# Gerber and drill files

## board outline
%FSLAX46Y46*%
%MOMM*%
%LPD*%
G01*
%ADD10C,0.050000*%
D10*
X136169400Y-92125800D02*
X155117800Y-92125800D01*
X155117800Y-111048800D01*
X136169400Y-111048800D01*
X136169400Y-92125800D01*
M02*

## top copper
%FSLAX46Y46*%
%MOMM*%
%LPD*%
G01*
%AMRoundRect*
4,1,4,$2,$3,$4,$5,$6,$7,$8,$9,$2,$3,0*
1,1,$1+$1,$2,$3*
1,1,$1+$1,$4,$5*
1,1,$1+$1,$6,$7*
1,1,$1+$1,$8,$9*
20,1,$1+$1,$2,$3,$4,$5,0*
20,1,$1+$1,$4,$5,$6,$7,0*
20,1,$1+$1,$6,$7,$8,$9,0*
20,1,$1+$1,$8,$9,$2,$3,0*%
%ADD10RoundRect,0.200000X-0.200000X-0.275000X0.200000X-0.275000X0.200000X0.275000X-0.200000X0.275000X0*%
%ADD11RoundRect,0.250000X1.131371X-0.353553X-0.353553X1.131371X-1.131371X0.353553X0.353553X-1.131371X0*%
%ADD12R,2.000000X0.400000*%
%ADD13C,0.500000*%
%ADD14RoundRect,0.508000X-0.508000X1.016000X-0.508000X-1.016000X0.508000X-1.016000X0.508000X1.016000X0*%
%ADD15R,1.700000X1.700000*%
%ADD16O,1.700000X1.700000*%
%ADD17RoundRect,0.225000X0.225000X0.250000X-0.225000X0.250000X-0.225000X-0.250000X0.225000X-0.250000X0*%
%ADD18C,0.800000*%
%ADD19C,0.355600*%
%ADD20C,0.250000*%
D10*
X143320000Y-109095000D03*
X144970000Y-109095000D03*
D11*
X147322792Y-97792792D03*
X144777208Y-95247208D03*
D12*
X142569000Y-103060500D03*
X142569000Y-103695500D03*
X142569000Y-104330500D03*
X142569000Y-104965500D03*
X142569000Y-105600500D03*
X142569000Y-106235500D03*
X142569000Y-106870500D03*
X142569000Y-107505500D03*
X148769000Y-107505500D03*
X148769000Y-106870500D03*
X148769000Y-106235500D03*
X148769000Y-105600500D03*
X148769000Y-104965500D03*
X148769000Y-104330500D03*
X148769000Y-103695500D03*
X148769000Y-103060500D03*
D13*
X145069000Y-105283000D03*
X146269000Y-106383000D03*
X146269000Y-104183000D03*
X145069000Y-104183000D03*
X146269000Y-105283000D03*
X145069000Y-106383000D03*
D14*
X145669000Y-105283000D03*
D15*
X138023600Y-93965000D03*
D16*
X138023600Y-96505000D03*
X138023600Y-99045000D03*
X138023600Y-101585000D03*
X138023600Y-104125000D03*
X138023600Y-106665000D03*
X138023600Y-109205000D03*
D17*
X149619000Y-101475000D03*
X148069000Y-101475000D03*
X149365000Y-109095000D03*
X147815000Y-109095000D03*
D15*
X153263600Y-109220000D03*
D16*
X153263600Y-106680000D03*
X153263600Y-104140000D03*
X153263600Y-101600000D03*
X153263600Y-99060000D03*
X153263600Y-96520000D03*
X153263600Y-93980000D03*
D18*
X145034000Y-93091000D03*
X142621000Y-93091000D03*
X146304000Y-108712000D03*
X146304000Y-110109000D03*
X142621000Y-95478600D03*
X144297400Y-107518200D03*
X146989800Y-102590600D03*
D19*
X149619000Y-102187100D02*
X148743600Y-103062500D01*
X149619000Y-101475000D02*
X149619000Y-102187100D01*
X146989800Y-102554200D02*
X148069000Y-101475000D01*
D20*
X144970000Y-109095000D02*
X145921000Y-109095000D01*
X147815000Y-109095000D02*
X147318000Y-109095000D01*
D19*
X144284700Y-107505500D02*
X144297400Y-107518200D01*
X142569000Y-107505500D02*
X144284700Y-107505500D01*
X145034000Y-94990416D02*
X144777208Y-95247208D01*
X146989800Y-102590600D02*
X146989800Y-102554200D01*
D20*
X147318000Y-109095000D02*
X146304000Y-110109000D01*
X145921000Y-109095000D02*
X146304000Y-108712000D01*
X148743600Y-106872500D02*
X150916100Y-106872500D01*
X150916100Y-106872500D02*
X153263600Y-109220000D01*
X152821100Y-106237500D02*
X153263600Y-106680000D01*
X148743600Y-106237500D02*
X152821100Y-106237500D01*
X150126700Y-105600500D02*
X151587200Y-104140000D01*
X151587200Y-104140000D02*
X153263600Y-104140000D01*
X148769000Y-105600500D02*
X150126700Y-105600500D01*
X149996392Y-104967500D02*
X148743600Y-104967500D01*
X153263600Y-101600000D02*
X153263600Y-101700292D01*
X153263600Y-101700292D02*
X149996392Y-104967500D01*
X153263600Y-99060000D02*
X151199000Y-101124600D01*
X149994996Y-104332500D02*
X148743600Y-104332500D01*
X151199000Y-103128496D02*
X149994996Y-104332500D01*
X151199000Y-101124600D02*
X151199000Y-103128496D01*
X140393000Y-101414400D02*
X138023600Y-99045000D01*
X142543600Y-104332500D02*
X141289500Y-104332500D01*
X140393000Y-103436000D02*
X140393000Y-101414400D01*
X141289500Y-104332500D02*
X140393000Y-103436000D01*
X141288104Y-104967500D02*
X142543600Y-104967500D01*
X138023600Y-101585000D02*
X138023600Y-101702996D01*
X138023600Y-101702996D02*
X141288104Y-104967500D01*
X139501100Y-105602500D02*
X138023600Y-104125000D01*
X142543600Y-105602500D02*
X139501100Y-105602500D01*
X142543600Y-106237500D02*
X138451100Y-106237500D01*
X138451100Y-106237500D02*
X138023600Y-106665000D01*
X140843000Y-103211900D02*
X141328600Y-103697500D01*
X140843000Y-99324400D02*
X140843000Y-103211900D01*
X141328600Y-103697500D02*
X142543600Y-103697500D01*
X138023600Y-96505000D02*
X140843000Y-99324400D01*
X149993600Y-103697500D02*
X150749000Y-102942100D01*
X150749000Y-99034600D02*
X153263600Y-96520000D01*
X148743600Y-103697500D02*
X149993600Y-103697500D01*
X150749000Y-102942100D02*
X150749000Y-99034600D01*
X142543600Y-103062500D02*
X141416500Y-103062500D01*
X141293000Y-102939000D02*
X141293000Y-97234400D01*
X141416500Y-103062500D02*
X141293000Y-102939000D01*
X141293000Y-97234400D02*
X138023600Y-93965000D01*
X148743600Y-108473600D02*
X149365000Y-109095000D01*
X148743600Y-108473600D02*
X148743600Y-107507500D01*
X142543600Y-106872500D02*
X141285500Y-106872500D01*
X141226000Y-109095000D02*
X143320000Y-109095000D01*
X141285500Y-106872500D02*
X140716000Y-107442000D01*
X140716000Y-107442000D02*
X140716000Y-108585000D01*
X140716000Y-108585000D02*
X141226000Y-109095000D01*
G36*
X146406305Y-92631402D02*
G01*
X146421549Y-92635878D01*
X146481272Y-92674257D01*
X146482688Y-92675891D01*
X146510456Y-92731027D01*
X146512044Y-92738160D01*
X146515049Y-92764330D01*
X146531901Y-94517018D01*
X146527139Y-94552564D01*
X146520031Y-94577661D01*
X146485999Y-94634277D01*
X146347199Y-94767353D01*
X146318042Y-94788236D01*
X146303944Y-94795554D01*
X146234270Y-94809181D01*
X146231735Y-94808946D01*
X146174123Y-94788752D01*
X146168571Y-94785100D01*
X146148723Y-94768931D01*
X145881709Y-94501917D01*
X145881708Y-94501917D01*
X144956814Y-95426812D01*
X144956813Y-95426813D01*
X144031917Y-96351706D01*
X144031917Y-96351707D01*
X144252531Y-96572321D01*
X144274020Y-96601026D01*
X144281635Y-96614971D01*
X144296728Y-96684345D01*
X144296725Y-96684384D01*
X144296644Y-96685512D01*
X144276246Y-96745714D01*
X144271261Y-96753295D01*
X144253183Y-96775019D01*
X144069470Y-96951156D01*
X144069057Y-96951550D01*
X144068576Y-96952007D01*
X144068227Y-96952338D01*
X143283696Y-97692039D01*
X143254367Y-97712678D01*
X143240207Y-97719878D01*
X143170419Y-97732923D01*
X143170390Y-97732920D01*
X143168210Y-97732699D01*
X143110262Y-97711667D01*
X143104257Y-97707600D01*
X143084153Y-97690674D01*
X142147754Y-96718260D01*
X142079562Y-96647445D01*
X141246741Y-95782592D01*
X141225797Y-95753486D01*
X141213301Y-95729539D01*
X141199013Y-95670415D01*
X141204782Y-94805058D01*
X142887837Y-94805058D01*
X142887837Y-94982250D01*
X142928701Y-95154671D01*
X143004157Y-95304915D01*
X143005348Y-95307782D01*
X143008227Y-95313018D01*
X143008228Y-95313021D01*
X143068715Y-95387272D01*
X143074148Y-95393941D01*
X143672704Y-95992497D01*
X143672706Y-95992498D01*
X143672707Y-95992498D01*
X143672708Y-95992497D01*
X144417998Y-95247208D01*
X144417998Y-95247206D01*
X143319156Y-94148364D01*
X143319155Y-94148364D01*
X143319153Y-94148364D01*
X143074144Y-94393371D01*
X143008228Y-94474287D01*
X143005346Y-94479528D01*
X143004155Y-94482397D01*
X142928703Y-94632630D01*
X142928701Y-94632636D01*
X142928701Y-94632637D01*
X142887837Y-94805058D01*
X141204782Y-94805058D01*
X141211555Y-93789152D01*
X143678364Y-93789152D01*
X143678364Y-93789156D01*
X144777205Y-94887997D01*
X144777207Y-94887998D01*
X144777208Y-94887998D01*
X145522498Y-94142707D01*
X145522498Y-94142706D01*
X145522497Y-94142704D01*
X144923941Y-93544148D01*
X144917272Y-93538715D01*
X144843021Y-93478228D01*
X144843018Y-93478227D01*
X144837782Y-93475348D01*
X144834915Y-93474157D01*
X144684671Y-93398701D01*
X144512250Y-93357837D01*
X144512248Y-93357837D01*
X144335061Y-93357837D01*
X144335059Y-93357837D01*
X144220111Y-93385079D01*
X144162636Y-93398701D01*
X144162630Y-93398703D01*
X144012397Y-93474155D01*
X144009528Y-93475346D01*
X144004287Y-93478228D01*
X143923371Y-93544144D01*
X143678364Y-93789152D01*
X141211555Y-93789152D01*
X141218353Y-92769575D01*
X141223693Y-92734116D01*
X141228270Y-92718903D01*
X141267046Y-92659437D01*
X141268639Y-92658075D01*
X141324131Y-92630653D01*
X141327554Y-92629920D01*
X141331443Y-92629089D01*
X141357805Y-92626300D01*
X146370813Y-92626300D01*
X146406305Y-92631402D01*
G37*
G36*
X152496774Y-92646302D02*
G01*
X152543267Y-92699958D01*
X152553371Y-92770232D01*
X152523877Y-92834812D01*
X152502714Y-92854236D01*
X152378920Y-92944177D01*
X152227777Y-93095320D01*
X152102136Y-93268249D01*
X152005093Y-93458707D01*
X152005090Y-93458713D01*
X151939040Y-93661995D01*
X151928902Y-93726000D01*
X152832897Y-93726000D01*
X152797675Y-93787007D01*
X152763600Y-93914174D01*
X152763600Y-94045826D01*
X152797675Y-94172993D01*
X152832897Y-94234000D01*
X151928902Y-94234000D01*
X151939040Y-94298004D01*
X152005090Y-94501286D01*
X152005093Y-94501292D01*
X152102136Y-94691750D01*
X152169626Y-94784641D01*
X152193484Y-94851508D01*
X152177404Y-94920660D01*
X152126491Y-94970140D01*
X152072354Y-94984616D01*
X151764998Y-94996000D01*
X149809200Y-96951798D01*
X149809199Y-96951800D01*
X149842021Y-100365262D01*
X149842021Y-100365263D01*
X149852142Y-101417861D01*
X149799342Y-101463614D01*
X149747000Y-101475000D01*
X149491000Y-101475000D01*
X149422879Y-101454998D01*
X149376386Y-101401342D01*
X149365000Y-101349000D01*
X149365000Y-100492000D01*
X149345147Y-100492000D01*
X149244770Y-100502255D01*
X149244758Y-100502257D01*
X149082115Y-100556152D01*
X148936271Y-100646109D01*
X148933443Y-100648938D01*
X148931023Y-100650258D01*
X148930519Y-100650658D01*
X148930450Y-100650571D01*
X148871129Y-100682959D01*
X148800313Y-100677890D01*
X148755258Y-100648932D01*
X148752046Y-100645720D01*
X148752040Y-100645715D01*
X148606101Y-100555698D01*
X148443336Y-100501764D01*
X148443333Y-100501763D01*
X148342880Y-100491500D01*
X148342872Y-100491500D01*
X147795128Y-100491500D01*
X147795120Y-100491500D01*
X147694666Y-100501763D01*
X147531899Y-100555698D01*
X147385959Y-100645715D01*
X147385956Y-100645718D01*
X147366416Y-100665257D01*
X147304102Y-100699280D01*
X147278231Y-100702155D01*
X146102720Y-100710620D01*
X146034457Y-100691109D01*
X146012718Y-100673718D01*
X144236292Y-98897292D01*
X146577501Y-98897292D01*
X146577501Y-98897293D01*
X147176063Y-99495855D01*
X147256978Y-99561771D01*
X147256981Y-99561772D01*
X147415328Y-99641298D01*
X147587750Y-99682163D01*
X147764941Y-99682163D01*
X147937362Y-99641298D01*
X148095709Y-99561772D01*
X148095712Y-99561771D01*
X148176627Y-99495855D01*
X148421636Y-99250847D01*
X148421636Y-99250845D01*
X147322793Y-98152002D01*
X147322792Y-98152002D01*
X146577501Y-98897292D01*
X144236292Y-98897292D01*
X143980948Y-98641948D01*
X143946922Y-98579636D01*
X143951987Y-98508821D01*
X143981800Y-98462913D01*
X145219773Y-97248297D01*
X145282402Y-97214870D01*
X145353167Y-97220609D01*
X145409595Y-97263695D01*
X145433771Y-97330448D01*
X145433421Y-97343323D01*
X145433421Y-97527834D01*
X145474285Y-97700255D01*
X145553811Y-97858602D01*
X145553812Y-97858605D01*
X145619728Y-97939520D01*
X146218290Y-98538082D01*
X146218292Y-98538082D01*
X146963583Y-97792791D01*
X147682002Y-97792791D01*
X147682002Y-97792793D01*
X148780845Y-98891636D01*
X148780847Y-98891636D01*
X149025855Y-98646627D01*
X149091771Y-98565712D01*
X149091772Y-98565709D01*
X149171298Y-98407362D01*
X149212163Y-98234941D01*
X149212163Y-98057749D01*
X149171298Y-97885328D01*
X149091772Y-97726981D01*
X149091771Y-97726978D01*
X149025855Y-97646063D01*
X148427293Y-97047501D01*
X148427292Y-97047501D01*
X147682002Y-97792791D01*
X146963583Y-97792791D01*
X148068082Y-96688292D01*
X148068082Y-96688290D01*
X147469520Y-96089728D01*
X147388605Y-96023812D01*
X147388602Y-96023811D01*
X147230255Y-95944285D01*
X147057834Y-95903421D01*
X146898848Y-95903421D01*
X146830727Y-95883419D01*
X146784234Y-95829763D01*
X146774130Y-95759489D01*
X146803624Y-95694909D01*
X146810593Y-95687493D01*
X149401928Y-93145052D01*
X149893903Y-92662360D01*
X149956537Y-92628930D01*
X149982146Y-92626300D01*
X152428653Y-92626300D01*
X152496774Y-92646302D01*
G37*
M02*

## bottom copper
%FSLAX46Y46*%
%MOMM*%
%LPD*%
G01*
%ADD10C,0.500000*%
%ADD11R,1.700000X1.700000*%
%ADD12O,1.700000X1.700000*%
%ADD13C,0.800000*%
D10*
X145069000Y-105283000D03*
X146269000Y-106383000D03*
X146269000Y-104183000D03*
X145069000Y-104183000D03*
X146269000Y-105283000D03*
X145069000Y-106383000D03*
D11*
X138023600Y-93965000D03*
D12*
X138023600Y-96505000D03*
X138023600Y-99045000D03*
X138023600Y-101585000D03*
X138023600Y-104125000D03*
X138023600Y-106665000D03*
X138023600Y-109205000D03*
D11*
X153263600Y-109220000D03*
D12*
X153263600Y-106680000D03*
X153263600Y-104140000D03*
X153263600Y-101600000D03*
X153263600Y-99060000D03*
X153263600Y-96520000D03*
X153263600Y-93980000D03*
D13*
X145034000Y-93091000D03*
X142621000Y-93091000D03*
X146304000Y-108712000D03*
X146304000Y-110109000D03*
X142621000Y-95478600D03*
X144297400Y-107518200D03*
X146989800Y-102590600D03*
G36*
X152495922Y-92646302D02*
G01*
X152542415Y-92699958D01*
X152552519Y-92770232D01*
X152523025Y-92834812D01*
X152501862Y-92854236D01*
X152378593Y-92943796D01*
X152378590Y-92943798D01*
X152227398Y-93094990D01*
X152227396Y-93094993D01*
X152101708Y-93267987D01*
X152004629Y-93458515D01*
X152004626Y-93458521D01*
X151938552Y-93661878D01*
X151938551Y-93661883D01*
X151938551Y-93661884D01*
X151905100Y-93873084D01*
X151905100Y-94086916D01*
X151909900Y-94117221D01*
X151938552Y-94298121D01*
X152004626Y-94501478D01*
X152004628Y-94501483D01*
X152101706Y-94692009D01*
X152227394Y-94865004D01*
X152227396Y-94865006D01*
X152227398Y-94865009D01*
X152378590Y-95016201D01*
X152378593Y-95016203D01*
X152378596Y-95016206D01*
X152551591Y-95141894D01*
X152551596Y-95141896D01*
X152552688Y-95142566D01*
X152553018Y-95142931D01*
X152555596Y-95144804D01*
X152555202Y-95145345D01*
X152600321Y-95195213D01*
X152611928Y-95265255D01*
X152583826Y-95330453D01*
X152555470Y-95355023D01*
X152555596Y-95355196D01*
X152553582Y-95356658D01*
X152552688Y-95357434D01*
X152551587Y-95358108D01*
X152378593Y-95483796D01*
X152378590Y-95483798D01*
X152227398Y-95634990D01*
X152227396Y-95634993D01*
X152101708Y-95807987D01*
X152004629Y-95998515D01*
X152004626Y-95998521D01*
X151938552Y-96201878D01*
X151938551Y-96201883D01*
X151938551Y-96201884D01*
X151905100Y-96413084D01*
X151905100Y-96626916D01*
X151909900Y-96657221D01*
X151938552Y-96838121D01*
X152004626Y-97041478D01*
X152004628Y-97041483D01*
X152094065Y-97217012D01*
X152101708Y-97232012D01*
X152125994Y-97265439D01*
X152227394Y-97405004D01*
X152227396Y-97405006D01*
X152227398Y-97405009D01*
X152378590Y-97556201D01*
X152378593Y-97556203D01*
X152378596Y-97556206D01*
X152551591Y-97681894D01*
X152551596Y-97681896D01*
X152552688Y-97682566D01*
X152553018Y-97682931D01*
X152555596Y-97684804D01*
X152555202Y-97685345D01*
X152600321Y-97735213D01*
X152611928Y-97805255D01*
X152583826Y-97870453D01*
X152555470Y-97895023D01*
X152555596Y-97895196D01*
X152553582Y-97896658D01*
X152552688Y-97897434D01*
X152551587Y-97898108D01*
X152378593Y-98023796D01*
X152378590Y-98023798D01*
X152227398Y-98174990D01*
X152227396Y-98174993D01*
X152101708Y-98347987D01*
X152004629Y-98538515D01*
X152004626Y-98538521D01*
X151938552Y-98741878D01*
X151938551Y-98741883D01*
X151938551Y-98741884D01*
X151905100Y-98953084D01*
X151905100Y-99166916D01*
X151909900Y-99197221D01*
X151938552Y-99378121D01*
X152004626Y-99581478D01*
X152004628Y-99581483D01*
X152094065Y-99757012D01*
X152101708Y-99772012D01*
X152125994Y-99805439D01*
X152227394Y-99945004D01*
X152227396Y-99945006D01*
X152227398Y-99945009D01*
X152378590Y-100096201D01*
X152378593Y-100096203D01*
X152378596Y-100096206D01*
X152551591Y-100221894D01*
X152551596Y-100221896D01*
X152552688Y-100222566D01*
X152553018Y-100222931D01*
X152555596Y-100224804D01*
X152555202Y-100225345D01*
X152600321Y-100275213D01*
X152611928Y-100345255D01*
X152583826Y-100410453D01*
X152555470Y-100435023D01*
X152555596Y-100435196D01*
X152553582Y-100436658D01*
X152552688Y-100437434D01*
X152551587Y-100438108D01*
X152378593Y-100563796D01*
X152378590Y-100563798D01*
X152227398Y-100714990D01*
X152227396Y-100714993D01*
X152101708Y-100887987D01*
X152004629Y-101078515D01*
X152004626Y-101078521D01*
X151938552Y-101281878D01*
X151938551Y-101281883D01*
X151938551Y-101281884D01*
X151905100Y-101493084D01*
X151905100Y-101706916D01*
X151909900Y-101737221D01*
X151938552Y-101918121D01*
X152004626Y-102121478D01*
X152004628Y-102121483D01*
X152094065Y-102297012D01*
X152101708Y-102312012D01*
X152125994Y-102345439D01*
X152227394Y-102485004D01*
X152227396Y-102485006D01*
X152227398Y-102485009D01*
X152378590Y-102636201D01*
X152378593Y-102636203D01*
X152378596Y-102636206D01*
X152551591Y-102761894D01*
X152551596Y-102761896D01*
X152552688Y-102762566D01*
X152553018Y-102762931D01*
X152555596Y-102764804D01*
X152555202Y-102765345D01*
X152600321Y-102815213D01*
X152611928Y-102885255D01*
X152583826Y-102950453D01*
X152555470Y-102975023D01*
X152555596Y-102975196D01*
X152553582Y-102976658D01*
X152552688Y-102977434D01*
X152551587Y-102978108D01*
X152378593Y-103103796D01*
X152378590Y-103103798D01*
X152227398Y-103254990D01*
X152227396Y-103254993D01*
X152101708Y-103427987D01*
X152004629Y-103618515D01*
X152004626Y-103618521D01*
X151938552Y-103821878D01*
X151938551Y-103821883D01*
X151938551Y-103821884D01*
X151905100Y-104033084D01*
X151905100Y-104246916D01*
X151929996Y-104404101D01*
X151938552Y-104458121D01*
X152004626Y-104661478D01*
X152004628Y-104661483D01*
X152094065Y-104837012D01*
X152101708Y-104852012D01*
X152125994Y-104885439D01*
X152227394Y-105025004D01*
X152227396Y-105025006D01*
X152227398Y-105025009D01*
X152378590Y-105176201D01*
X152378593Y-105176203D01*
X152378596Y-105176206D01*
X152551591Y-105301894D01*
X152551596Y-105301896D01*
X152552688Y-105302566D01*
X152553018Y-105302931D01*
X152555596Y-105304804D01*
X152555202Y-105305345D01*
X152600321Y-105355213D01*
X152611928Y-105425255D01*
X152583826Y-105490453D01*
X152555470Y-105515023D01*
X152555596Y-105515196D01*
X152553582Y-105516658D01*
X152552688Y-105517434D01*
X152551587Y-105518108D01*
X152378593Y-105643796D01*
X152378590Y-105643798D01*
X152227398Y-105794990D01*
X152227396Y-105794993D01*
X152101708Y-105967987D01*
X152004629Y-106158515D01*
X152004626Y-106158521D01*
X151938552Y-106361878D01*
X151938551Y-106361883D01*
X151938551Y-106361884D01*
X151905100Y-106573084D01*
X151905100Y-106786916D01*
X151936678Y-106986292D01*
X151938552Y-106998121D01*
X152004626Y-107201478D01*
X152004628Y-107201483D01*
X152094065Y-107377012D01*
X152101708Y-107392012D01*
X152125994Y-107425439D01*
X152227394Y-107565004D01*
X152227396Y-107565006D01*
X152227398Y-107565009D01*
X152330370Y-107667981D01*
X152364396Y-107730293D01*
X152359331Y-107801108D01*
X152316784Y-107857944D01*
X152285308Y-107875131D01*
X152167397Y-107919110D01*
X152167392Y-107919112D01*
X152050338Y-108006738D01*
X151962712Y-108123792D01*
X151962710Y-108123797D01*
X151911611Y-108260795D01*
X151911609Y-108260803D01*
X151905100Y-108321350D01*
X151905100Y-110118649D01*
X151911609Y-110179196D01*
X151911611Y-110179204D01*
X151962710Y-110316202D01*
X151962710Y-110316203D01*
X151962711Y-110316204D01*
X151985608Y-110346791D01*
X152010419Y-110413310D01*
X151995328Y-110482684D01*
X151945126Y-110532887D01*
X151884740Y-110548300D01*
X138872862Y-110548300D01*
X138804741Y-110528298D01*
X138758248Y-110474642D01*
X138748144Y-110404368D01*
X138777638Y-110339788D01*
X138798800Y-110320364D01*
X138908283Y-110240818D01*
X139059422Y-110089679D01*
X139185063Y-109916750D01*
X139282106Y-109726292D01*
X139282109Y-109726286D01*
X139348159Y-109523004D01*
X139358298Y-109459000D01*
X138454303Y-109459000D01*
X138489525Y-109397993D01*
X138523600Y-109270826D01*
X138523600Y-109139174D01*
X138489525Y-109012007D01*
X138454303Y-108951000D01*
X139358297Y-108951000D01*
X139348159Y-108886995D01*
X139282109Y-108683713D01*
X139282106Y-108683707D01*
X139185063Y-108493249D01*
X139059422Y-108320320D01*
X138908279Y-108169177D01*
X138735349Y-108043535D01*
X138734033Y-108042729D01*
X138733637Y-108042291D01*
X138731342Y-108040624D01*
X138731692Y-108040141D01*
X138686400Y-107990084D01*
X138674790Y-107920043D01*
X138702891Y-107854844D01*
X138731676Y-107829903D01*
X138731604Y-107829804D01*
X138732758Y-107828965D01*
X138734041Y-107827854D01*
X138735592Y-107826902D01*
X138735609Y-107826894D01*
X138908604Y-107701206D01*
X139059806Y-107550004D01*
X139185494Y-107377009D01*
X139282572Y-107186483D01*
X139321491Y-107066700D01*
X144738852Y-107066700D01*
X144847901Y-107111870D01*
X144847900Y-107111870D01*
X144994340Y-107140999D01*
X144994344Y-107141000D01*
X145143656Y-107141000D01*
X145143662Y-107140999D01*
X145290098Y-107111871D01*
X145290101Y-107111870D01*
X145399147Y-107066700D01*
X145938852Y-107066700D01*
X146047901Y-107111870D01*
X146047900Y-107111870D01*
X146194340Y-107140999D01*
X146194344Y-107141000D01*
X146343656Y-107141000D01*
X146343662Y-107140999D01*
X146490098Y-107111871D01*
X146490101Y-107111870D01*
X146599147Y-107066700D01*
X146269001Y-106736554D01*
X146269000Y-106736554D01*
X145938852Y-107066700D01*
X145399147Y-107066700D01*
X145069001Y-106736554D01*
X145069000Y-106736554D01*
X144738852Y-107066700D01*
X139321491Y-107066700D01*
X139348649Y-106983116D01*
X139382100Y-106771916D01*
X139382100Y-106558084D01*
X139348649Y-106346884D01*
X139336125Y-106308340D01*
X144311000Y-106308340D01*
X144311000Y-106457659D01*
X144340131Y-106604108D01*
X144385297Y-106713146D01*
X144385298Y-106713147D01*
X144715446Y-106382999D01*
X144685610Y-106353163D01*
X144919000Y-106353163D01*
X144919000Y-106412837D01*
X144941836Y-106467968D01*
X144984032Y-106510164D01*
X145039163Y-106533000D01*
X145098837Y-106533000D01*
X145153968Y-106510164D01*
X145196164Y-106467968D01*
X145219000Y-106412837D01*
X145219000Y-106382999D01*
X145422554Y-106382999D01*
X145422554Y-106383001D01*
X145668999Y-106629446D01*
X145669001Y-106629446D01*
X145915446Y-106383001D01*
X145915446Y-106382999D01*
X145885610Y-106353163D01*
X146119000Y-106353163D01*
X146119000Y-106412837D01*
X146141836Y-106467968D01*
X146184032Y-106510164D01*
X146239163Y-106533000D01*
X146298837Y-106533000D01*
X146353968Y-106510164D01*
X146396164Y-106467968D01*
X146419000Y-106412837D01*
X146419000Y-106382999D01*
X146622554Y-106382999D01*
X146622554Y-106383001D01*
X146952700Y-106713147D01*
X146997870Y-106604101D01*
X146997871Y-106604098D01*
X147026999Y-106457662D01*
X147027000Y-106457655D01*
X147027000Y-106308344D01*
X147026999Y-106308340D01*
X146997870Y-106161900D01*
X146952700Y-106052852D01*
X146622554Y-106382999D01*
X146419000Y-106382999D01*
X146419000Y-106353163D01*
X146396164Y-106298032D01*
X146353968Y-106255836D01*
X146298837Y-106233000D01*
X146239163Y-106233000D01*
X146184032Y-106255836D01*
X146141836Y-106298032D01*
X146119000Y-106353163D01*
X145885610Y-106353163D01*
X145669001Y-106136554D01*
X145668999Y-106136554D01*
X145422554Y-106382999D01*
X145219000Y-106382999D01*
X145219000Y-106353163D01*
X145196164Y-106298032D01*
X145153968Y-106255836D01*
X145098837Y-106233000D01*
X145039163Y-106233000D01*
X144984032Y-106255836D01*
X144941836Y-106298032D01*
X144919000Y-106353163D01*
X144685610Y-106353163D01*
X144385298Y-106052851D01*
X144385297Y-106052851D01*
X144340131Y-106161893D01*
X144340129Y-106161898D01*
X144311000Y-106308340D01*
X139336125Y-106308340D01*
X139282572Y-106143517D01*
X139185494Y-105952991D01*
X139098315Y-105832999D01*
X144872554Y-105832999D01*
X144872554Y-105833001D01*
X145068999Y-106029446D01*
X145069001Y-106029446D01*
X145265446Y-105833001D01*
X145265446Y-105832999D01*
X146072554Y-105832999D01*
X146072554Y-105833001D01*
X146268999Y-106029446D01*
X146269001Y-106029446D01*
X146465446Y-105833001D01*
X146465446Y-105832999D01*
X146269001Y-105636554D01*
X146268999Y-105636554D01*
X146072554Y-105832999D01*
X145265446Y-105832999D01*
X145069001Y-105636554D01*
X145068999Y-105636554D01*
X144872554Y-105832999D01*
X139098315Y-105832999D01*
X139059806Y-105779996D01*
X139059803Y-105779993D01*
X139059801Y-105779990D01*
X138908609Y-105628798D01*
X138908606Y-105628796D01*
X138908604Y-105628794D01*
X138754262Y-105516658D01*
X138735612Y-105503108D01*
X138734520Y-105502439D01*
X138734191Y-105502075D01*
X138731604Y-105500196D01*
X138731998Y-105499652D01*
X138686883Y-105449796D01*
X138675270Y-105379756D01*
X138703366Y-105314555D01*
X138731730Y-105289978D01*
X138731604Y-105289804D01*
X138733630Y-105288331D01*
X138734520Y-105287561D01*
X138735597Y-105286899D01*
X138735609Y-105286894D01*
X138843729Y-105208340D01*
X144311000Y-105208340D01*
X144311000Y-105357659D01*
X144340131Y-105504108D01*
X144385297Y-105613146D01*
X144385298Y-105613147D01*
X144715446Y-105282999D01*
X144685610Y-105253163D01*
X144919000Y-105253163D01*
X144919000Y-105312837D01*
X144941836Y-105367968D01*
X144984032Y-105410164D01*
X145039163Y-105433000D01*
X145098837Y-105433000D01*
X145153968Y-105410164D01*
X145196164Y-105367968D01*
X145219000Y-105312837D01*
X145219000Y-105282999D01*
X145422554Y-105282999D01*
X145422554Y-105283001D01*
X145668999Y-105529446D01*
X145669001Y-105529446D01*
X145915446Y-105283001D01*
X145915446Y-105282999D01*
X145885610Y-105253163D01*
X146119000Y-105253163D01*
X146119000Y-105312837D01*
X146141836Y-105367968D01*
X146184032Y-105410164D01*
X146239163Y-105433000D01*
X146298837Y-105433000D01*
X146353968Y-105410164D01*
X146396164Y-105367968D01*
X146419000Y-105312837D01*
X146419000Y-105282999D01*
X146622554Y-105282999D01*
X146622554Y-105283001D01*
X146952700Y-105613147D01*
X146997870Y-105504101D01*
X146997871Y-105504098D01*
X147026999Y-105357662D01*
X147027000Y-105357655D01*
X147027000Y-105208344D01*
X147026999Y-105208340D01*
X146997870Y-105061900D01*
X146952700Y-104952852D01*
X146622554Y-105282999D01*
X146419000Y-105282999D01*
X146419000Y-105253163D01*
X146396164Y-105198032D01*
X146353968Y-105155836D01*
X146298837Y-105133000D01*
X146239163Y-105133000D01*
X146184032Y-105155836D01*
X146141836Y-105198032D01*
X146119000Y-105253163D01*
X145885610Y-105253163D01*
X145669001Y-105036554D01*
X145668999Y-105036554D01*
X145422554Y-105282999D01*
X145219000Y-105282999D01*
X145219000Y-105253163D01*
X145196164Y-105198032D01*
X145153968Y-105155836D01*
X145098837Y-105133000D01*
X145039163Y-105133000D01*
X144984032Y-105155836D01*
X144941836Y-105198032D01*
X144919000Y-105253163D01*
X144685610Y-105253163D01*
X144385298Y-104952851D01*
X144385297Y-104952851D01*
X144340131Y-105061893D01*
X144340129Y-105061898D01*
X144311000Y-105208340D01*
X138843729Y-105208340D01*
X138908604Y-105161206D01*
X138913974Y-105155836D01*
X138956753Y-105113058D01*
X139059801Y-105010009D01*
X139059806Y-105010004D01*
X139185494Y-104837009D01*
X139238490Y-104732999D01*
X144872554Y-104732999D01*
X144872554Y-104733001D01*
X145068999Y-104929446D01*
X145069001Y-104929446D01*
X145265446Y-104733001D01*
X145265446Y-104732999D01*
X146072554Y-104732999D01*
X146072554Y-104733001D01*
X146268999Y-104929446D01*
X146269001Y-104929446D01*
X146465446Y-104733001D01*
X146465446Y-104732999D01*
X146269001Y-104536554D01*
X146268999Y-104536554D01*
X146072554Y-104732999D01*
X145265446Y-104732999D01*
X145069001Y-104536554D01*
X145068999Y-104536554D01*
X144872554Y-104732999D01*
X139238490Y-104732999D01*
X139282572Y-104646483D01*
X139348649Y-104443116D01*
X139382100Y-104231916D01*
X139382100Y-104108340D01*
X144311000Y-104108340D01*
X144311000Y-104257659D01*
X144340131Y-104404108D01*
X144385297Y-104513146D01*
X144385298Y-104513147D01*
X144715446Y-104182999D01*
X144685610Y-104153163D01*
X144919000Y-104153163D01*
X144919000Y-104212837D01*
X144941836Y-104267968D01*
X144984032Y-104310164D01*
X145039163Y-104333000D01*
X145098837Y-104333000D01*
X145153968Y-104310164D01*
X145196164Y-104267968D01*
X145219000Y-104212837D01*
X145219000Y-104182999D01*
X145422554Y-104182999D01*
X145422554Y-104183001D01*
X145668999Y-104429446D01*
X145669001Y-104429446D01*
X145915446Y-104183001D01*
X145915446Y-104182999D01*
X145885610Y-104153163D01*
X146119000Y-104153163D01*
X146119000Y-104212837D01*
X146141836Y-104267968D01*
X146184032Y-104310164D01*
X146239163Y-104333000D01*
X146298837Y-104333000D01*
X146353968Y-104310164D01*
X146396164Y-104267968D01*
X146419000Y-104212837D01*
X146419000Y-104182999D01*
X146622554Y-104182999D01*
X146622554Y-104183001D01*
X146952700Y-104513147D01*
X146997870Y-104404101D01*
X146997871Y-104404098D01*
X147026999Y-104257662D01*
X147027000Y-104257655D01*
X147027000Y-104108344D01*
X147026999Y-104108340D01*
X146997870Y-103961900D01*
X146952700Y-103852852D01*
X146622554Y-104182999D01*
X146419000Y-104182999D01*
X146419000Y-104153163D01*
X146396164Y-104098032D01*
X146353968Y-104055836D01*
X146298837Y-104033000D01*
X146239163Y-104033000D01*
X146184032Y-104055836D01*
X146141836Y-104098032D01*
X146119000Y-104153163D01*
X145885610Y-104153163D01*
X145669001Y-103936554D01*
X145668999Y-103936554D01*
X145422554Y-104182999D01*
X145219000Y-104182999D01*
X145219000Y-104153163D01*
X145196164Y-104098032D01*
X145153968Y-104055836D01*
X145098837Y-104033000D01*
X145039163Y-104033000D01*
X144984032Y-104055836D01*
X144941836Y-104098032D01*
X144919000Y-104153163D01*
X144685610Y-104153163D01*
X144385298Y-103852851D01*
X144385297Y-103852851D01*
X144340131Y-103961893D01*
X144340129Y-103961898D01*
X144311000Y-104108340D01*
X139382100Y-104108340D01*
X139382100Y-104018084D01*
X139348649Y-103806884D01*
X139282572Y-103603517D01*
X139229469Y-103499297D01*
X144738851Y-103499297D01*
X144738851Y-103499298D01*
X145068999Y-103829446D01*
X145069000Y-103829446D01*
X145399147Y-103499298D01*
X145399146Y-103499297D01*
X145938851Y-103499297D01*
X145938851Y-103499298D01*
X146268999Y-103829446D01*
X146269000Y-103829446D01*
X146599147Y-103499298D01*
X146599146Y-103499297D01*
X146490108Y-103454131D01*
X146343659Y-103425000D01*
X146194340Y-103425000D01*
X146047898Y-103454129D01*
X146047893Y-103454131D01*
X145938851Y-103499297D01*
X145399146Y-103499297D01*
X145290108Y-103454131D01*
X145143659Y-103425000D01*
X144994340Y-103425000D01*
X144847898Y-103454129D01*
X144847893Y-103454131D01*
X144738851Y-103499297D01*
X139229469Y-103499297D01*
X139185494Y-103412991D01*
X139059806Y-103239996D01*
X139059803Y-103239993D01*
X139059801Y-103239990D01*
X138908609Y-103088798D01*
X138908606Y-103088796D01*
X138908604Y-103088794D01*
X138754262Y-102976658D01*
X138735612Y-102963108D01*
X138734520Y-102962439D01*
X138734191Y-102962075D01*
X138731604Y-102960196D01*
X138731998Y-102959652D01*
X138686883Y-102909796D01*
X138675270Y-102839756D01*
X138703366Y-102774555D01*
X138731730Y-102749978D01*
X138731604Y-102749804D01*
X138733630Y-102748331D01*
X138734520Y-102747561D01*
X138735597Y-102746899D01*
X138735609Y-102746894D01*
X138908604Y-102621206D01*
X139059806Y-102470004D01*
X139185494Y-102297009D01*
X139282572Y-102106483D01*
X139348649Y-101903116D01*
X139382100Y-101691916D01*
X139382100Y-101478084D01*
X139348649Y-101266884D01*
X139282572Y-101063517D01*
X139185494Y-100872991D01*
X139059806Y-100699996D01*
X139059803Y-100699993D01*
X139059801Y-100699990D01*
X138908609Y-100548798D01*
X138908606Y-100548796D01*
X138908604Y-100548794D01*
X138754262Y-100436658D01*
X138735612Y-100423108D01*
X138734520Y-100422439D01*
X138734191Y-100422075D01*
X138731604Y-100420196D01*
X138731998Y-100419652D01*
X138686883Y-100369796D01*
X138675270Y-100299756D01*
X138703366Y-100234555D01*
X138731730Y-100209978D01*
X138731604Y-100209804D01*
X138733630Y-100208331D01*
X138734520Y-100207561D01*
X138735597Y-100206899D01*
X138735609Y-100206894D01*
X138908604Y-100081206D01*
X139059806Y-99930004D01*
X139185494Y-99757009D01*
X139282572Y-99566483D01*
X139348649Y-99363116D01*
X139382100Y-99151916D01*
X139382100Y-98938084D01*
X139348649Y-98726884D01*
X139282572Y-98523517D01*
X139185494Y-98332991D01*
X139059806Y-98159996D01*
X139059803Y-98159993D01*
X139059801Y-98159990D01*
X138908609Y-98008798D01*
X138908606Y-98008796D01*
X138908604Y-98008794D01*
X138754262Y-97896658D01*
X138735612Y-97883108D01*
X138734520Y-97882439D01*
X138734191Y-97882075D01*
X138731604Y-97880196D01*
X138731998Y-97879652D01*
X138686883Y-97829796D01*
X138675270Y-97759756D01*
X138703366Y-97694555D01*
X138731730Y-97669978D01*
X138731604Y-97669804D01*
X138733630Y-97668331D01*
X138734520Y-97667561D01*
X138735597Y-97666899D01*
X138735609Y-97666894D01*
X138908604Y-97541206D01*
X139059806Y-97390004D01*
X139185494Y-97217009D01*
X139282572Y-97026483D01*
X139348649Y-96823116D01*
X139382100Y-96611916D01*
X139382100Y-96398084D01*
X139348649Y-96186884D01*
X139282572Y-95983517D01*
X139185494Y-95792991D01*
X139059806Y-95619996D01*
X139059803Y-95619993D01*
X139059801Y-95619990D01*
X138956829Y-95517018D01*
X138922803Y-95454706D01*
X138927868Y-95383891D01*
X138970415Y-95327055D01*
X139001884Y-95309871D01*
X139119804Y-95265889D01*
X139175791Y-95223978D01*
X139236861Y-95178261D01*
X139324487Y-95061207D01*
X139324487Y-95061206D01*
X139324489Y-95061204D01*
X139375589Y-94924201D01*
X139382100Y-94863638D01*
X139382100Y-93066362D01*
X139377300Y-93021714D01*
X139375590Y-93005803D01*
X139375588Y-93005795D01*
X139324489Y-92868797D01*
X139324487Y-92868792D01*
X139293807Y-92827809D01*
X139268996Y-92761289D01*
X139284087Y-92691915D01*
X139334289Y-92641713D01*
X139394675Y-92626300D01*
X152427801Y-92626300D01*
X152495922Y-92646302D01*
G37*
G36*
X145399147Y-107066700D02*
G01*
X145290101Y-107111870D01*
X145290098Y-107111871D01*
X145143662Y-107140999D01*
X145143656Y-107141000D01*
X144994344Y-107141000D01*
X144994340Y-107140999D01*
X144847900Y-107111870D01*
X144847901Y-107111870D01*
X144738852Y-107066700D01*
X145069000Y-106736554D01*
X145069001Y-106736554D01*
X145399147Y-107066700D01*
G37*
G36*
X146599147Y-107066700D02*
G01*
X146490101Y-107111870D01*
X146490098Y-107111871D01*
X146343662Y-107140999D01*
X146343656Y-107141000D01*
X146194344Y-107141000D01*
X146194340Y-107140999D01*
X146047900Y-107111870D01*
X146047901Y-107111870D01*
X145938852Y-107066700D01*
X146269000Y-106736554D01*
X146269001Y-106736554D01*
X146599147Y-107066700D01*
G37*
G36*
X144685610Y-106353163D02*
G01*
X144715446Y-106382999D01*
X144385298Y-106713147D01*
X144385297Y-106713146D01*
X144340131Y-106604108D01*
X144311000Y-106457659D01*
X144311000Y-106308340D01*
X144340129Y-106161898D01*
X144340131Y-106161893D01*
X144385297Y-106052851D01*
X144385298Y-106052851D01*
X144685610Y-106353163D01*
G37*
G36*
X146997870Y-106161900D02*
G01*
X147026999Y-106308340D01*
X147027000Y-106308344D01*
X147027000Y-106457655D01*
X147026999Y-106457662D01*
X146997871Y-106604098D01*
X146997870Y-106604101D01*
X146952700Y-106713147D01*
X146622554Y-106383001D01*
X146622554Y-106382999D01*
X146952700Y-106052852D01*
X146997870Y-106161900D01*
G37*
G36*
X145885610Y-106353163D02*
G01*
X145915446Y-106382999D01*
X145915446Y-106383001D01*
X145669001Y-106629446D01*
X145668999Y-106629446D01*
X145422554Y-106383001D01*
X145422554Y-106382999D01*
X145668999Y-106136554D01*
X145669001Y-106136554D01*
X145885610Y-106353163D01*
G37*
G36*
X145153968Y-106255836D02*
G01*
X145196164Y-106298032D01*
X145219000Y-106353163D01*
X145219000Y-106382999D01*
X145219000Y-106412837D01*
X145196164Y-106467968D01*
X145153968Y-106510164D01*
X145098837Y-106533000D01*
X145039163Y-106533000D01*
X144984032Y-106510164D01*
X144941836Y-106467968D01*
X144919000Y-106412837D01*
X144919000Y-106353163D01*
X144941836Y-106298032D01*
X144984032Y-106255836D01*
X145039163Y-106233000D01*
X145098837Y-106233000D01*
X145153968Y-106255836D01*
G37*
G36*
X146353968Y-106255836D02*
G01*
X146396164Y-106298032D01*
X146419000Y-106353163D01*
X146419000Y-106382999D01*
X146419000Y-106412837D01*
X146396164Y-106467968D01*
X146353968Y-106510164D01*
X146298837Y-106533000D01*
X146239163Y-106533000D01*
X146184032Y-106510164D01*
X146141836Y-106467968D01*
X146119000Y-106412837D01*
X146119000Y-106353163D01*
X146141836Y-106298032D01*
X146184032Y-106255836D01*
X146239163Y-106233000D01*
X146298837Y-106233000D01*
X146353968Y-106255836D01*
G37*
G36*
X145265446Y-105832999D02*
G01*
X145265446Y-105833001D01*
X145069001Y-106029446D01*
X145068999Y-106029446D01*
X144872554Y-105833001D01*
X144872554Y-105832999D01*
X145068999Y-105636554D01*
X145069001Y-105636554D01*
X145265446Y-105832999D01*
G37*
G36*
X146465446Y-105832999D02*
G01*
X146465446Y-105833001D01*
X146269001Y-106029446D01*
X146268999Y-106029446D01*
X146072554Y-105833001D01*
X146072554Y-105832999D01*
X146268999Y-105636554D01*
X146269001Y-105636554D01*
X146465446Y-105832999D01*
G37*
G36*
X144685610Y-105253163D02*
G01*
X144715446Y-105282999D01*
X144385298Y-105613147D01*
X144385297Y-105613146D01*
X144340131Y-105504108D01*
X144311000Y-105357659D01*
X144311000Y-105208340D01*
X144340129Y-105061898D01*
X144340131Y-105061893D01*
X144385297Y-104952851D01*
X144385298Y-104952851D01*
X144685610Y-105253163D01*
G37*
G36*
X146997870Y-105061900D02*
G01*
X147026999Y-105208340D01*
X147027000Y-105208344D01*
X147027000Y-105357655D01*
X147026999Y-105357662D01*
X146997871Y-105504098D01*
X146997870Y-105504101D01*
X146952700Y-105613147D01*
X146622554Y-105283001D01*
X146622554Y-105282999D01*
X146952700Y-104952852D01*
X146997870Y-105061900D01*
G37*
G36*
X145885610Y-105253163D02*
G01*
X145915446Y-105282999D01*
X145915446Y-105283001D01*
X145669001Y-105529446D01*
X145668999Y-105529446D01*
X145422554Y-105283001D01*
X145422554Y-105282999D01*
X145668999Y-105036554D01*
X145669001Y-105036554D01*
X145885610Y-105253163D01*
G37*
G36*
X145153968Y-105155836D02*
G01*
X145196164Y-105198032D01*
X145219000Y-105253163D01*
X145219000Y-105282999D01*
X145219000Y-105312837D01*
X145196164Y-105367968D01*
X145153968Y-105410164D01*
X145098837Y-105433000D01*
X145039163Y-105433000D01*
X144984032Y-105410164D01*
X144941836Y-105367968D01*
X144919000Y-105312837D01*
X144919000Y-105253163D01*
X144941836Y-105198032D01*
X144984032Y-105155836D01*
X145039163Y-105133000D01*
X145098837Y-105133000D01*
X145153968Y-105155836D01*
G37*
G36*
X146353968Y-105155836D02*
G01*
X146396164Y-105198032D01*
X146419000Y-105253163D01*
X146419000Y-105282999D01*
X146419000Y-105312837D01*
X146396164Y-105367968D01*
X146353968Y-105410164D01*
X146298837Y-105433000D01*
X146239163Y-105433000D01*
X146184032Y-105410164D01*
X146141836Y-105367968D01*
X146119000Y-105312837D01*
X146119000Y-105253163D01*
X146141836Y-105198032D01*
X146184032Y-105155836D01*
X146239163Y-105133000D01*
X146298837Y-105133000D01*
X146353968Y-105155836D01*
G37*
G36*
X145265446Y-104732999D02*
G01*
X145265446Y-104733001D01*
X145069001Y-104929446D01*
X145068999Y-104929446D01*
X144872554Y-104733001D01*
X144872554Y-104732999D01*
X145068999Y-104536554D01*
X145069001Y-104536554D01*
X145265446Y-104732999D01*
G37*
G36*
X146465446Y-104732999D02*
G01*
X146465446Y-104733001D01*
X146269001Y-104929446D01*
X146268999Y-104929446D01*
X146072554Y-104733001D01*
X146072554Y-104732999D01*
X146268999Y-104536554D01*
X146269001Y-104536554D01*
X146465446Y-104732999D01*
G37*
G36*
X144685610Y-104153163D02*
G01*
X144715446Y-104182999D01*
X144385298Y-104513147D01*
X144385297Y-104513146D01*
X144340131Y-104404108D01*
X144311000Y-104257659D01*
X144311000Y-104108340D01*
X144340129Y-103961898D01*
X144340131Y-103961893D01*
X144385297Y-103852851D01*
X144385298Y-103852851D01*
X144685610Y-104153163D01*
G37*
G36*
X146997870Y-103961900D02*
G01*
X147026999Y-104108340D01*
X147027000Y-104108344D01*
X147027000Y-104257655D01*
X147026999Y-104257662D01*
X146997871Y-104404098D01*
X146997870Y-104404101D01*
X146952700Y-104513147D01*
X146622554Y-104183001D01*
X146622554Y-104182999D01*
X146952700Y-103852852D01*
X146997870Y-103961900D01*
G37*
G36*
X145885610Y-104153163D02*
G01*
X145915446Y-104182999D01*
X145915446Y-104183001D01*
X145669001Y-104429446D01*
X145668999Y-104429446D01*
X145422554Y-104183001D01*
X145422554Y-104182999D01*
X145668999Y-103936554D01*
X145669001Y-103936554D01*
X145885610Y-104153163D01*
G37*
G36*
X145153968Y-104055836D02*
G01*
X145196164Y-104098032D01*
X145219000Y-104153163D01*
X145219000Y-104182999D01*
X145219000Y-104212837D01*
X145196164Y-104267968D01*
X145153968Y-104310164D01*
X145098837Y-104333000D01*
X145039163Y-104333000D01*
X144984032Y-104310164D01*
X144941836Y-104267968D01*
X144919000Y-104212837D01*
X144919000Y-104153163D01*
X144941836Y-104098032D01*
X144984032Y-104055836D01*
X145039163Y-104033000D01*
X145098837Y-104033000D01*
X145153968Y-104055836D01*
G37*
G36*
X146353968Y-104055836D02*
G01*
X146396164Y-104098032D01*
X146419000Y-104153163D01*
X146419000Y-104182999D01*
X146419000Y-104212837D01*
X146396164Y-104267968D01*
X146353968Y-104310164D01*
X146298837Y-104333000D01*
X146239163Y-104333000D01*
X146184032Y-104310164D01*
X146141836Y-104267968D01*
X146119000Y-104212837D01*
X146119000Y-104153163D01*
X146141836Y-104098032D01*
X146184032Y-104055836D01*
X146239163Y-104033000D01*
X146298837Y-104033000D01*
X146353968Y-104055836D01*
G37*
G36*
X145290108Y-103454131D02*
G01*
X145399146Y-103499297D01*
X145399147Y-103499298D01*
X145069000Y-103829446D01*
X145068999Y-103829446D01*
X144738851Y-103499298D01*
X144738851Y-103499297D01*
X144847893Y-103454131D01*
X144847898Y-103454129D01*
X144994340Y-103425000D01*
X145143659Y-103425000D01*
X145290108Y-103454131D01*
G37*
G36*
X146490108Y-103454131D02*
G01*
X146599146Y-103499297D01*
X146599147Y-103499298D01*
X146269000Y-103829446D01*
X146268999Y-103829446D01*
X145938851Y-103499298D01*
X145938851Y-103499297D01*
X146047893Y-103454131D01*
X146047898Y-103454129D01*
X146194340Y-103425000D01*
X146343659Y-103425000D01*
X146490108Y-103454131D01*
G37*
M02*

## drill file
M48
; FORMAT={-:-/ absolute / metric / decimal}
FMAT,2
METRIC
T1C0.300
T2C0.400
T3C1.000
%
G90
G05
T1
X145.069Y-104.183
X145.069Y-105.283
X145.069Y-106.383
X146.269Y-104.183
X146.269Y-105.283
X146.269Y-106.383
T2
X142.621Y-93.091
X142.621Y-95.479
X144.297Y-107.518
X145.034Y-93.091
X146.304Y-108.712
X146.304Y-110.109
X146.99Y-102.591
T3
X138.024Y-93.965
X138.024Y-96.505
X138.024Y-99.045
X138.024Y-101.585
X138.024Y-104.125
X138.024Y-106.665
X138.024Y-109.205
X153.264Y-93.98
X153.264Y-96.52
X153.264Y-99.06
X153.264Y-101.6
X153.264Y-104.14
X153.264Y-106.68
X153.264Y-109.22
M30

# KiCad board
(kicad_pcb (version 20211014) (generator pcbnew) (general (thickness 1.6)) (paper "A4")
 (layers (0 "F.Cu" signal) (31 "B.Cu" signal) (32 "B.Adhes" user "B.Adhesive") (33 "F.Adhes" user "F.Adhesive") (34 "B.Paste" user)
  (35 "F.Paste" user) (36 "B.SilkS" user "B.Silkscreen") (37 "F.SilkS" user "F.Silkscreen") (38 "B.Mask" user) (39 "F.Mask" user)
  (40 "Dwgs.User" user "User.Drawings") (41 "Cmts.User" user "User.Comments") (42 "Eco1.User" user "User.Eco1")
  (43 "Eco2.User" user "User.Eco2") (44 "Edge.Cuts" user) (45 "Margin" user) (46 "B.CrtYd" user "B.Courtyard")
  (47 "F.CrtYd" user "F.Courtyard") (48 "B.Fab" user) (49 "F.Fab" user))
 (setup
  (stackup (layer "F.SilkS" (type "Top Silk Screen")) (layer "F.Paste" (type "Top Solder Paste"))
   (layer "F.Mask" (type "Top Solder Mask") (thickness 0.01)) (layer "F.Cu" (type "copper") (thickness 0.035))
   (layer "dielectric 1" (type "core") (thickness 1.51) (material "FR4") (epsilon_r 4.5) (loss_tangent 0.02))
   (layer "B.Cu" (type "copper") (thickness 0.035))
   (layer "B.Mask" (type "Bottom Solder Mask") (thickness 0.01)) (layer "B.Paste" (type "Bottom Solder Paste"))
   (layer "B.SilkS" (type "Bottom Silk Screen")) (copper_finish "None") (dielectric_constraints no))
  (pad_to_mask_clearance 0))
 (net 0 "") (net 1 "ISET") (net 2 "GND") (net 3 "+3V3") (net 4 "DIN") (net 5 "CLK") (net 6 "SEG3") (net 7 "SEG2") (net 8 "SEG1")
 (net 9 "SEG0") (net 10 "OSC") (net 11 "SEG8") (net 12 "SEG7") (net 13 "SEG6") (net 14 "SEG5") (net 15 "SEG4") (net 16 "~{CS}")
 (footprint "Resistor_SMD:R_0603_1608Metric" (layer "F.Cu") (at 144.145 109.095)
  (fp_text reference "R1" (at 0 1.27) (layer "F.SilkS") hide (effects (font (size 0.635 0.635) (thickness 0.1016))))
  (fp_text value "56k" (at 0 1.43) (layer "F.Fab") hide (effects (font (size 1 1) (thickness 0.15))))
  (pad "1" smd roundrect (at -0.825 0) (size 0.8 0.95) (layers "F.Cu" "F.Paste" "F.Mask") (roundrect_rratio 0.25) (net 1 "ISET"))
  (pad "2" smd roundrect (at 0.825 0) (size 0.8 0.95) (layers "F.Cu" "F.Paste" "F.Mask") (roundrect_rratio 0.25) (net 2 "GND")))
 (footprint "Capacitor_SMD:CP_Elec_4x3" (layer "F.Cu") (at 146.05 96.52 135)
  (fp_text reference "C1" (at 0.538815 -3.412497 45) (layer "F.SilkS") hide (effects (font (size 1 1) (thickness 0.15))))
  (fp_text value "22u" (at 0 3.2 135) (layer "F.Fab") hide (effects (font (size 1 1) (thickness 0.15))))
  (pad "1" smd roundrect (at -1.8 0 135) (size 2.6 1.6) (layers "F.Cu" "F.Paste" "F.Mask") (roundrect_rratio 0.15625) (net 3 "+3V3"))
  (pad "2" smd roundrect (at 1.8 0 135) (size 2.6 1.6) (layers "F.Cu" "F.Paste" "F.Mask") (roundrect_rratio 0.15625) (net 2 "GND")))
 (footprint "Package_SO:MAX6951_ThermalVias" (layer "F.Cu") (at 145.669 105.283 -90)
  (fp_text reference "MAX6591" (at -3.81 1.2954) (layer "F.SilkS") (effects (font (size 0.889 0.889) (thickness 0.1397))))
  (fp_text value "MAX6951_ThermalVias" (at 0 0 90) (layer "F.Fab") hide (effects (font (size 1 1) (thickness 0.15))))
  (pad "1" smd rect (at -2.2225 3.1 270) (size 0.4 2) (layers "F.Cu" "F.Paste" "F.Mask") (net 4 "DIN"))
  (pad "2" smd rect (at -1.5875 3.1 270) (size 0.4 2) (layers "F.Cu" "F.Paste" "F.Mask") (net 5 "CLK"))
  (pad "3" smd rect (at -0.9525 3.1 270) (size 0.4 2) (layers "F.Cu" "F.Paste" "F.Mask") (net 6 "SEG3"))
  (pad "4" smd rect (at -0.3175 3.1 270) (size 0.4 2) (layers "F.Cu" "F.Paste" "F.Mask") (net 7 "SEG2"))
  (pad "5" smd rect (at 0.3175 3.1 270) (size 0.4 2) (layers "F.Cu" "F.Paste" "F.Mask") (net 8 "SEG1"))
  (pad "6" smd rect (at 0.9525 3.1 270) (size 0.4 2) (layers "F.Cu" "F.Paste" "F.Mask") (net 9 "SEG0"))
  (pad "7" smd rect (at 1.5875 3.1 270) (size 0.4 2) (layers "F.Cu" "F.Paste" "F.Mask") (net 1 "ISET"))
  (pad "8" smd rect (at 2.2225 3.1 270) (size 0.4 2) (layers "F.Cu" "F.Paste" "F.Mask") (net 2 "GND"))
  (pad "9" smd rect (at 2.2225 -3.1 270) (size 0.4 2) (layers "F.Cu" "F.Paste" "F.Mask") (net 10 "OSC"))
  (pad "10" smd rect (at 1.5875 -3.1 270) (size 0.4 2) (layers "F.Cu" "F.Paste" "F.Mask") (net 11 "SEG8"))
  (pad "11" smd rect (at 0.9525 -3.1 270) (size 0.4 2) (layers "F.Cu" "F.Paste" "F.Mask") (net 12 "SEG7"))
  (pad "12" smd rect (at 0.3175 -3.1 270) (size 0.4 2) (layers "F.Cu" "F.Paste" "F.Mask") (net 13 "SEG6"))
  (pad "13" smd rect (at -0.3175 -3.1 270) (size 0.4 2) (layers "F.Cu" "F.Paste" "F.Mask") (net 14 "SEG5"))
  (pad "14" smd rect (at -0.9525 -3.1 270) (size 0.4 2) (layers "F.Cu" "F.Paste" "F.Mask") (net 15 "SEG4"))
  (pad "15" smd rect (at -1.5875 -3.1 270) (size 0.4 2) (layers "F.Cu" "F.Paste" "F.Mask") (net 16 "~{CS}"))
  (pad "16" smd rect (at -2.2225 -3.1 270) (size 0.4 2) (layers "F.Cu" "F.Paste" "F.Mask") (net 3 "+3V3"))
  (pad "17" thru_hole circle (at 0 0.6 270) (size 0.5 0.5) (drill 0.3) (layers *.Cu) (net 2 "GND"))
  (pad "17" thru_hole circle (at 1.1 -0.6 270) (size 0.5 0.5) (drill 0.3) (layers *.Cu) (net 2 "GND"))
  (pad "17" thru_hole circle (at -1.1 -0.6 270) (size 0.5 0.5) (drill 0.3) (layers *.Cu) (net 2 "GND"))
  (pad "17" thru_hole circle (at -1.1 0.6 270) (size 0.5 0.5) (drill 0.3) (layers *.Cu) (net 2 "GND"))
  (pad "17" thru_hole circle (at 0 -0.6 270) (size 0.5 0.5) (drill 0.3) (layers *.Cu) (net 2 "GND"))
  (pad "17" thru_hole circle (at 1.1 0.6 270) (size 0.5 0.5) (drill 0.3) (layers *.Cu) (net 2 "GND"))
  (pad "17" smd roundrect (at 0 0 270) (size 3.048 2.032) (layers "F.Cu" "F.Paste" "F.Mask") (roundrect_rratio 0.25) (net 2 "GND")))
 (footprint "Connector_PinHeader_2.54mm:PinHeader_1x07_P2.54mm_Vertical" (layer "F.Cu") (at 138.0236 93.965)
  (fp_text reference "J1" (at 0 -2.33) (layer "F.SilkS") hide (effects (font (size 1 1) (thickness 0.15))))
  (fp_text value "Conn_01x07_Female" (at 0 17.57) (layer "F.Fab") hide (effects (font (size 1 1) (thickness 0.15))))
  (pad "1" thru_hole rect (at 0 0) (size 1.7 1.7) (drill 1) (layers *.Cu *.Mask) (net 4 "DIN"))
  (pad "2" thru_hole oval (at 0 2.54) (size 1.7 1.7) (drill 1) (layers *.Cu *.Mask) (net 5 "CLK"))
  (pad "3" thru_hole oval (at 0 5.08) (size 1.7 1.7) (drill 1) (layers *.Cu *.Mask) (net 6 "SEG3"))
  (pad "4" thru_hole oval (at 0 7.62) (size 1.7 1.7) (drill 1) (layers *.Cu *.Mask) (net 7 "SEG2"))
  (pad "5" thru_hole oval (at 0 10.16) (size 1.7 1.7) (drill 1) (layers *.Cu *.Mask) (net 8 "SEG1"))
  (pad "6" thru_hole oval (at 0 12.7) (size 1.7 1.7) (drill 1) (layers *.Cu *.Mask) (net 9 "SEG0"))
  (pad "7" thru_hole oval (at 0 15.24) (size 1.7 1.7) (drill 1) (layers *.Cu *.Mask) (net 2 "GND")))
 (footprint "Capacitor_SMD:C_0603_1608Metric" (layer "F.Cu") (at 148.844 101.475 180)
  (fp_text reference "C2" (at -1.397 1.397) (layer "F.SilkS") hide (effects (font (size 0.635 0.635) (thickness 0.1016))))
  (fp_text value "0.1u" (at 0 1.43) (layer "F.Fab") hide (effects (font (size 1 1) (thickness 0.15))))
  (pad "1" smd roundrect (at -0.775 0 180) (size 0.9 0.95) (layers "F.Cu" "F.Paste" "F.Mask") (roundrect_rratio 0.25) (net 3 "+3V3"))
  (pad "2" smd roundrect (at 0.775 0 180) (size 0.9 0.95) (layers "F.Cu" "F.Paste" "F.Mask") (roundrect_rratio 0.25) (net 2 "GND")))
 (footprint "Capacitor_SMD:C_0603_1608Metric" (layer "F.Cu") (at 148.59 109.095 180)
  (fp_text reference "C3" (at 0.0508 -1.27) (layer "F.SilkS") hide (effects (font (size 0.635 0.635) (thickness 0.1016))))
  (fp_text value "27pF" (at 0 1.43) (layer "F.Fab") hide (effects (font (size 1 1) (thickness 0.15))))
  (pad "1" smd roundrect (at -0.775 0 180) (size 0.9 0.95) (layers "F.Cu" "F.Paste" "F.Mask") (roundrect_rratio 0.25) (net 10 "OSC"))
  (pad "2" smd roundrect (at 0.775 0 180) (size 0.9 0.95) (layers "F.Cu" "F.Paste" "F.Mask") (roundrect_rratio 0.25) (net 2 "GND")))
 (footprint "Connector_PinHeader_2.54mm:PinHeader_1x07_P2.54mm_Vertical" (layer "F.Cu") (at 153.2636 109.22 180)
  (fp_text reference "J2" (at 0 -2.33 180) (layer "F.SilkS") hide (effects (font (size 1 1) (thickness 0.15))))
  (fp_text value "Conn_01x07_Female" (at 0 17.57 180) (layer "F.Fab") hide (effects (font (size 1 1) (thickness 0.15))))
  (pad "1" thru_hole rect (at 0 0 180) (size 1.7 1.7) (drill 1) (layers *.Cu *.Mask) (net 11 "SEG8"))
  (pad "2" thru_hole oval (at 0 2.54 180) (size 1.7 1.7) (drill 1) (layers *.Cu *.Mask) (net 12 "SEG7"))
  (pad "3" thru_hole oval (at 0 5.08 180) (size 1.7 1.7) (drill 1) (layers *.Cu *.Mask) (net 13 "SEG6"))
  (pad "4" thru_hole oval (at 0 7.62 180) (size 1.7 1.7) (drill 1) (layers *.Cu *.Mask) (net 14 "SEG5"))
  (pad "5" thru_hole oval (at 0 10.16 180) (size 1.7 1.7) (drill 1) (layers *.Cu *.Mask) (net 15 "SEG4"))
  (pad "6" thru_hole oval (at 0 12.7 180) (size 1.7 1.7) (drill 1) (layers *.Cu *.Mask) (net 16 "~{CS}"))
  (pad "7" thru_hole oval (at 0 15.24 180) (size 1.7 1.7) (drill 1) (layers *.Cu *.Mask) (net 3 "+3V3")))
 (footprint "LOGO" (layer "B.Cu") (at 142.586948 101.043132 -90)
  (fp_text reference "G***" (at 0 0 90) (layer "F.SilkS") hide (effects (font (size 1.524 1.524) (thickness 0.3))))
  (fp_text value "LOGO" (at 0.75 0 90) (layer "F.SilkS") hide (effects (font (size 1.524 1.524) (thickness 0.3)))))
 (gr_rect (start 136.1694 92.1258) (end 155.1178 111.0488) (layer "Edge.Cuts") (width 0.05) (fill none))
 (segment (start 149.619 102.1871) (end 148.7436 103.0625) (width 0.3556) (layer "F.Cu") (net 3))
 (segment (start 149.619 101.475) (end 149.619 102.1871) (width 0.3556) (layer "F.Cu") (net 3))
 (segment (start 146.9898 102.5542) (end 148.069 101.475) (width 0.3556) (layer "F.Cu") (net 2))
 (segment (start 144.97 109.095) (end 145.921 109.095) (width 0.25) (layer "F.Cu") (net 2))
 (segment (start 147.815 109.095) (end 147.318 109.095) (width 0.25) (layer "F.Cu") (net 2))
 (segment (start 144.2847 107.5055) (end 144.2974 107.5182) (width 0.3556) (layer "F.Cu") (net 2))
 (segment (start 142.569 107.5055) (end 144.2847 107.5055) (width 0.3556) (layer "F.Cu") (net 2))
 (segment (start 145.034 94.990416) (end 144.777208 95.247208) (width 0.3556) (layer "F.Cu") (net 2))
 (segment (start 146.9898 102.5906) (end 146.9898 102.5542) (width 0.3556) (layer "F.Cu") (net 2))
 (segment (start 147.318 109.095) (end 146.304 110.109) (width 0.25) (layer "F.Cu") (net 2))
 (segment (start 145.921 109.095) (end 146.304 108.712) (width 0.25) (layer "F.Cu") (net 2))
 (via (at 145.034 93.091) (size 0.8) (drill 0.4) (layers "F.Cu" "B.Cu") (free) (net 2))
 (via (at 142.621 93.091) (size 0.8) (drill 0.4) (layers "F.Cu" "B.Cu") (free) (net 2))
 (via (at 146.304 108.712) (size 0.8) (drill 0.4) (layers "F.Cu" "B.Cu") (free) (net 2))
 (via (at 146.304 110.109) (size 0.8) (drill 0.4) (layers "F.Cu" "B.Cu") (free) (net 2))
 (via (at 142.621 95.4786) (size 0.8) (drill 0.4) (layers "F.Cu" "B.Cu") (free) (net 2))
 (via (at 144.2974 107.5182) (size 0.8) (drill 0.4) (layers "F.Cu" "B.Cu") (free) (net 2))
 (via (at 146.9898 102.5906) (size 0.8) (drill 0.4) (layers "F.Cu" "B.Cu") (free) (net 2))
 (segment (start 148.7436 106.8725) (end 150.9161 106.8725) (width 0.25) (layer "F.Cu") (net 11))
 (segment (start 150.9161 106.8725) (end 153.2636 109.22) (width 0.25) (layer "F.Cu") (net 11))
 (segment (start 152.8211 106.2375) (end 153.2636 106.68) (width 0.25) (layer "F.Cu") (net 12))
 (segment (start 148.7436 106.2375) (end 152.8211 106.2375) (width 0.25) (layer "F.Cu") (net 12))
 (segment (start 150.1267 105.6005) (end 151.5872 104.14) (width 0.25) (layer "F.Cu") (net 13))
 (segment (start 151.5872 104.14) (end 153.2636 104.14) (width 0.25) (layer "F.Cu") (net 13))
 (segment (start 148.769 105.6005) (end 150.1267 105.6005) (width 0.25) (layer "F.Cu") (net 13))
 (segment (start 149.996392 104.9675) (end 148.7436 104.9675) (width 0.25) (layer "F.Cu") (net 14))
 (segment (start 153.2636 101.6) (end 153.2636 101.700292) (width 0.25) (layer "F.Cu") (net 14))
 (segment (start 153.2636 101.700292) (end 149.996392 104.9675) (width 0.25) (layer "F.Cu") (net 14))
 (segment (start 153.2636 99.06) (end 151.199 101.1246) (width 0.25) (layer "F.Cu") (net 15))
 (segment (start 149.994996 104.3325) (end 148.7436 104.3325) (width 0.25) (layer "F.Cu") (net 15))
 (segment (start 151.199 103.128496) (end 149.994996 104.3325) (width 0.25) (layer "F.Cu") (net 15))
 (segment (start 151.199 101.1246) (end 151.199 103.128496) (width 0.25) (layer "F.Cu") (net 15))
 (segment (start 140.393 101.4144) (end 138.0236 99.045) (width 0.25) (layer "F.Cu") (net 6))
 (segment (start 142.5436 104.3325) (end 141.2895 104.3325) (width 0.25) (layer "F.Cu") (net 6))
 (segment (start 140.393 103.436) (end 140.393 101.4144) (width 0.25) (layer "F.Cu") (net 6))
 (segment (start 141.2895 104.3325) (end 140.393 103.436) (width 0.25) (layer "F.Cu") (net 6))
 (segment (start 141.288104 104.9675) (end 142.5436 104.9675) (width 0.25) (layer "F.Cu") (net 7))
 (segment (start 138.0236 101.585) (end 138.0236 101.702996) (width 0.25) (layer "F.Cu") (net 7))
 (segment (start 138.0236 101.702996) (end 141.288104 104.9675) (width 0.25) (layer "F.Cu") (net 7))
 (segment (start 139.5011 105.6025) (end 138.0236 104.125) (width 0.25) (layer "F.Cu") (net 8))
 (segment (start 142.5436 105.6025) (end 139.5011 105.6025) (width 0.25) (layer "F.Cu") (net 8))
 (segment (start 142.5436 106.2375) (end 138.4511 106.2375) (width 0.25) (layer "F.Cu") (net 9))
 (segment (start 138.4511 106.2375) (end 138.0236 106.665) (width 0.25) (layer "F.Cu") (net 9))
 (segment (start 140.843 103.2119) (end 141.3286 103.6975) (width 0.25) (layer "F.Cu") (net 5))
 (segment (start 140.843 99.3244) (end 140.843 103.2119) (width 0.25) (layer "F.Cu") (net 5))
 (segment (start 141.3286 103.6975) (end 142.5436 103.6975) (width 0.25) (layer "F.Cu") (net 5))
 (segment (start 138.0236 96.505) (end 140.843 99.3244) (width 0.25) (layer "F.Cu") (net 5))
 (segment (start 149.9936 103.6975) (end 150.749 102.9421) (width 0.25) (layer "F.Cu") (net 16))
 (segment (start 150.749 99.0346) (end 153.2636 96.52) (width 0.25) (layer "F.Cu") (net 16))
 (segment (start 148.7436 103.6975) (end 149.9936 103.6975) (width 0.25) (layer "F.Cu") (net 16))
 (segment (start 150.749 102.9421) (end 150.749 99.0346) (width 0.25) (layer "F.Cu") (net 16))
 (segment (start 142.5436 103.0625) (end 141.4165 103.0625) (width 0.25) (layer "F.Cu") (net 4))
 (segment (start 141.293 102.939) (end 141.293 97.2344) (width 0.25) (layer "F.Cu") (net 4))
 (segment (start 141.4165 103.0625) (end 141.293 102.939) (width 0.25) (layer "F.Cu") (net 4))
 (segment (start 141.293 97.2344) (end 138.0236 93.965) (width 0.25) (layer "F.Cu") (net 4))
 (segment (start 148.7436 108.4736) (end 149.365 109.095) (width 0.25) (layer "F.Cu") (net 10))
 (segment (start 148.7436 108.4736) (end 148.7436 107.5075) (width 0.25) (layer "F.Cu") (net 10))
 (segment (start 142.5436 106.8725) (end 141.2855 106.8725) (width 0.25) (layer "F.Cu") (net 1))
 (segment (start 141.226 109.095) (end 143.32 109.095) (width 0.25) (layer "F.Cu") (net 1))
 (segment (start 141.2855 106.8725) (end 140.716 107.442) (width 0.25) (layer "F.Cu") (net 1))
 (segment (start 140.716 107.442) (end 140.716 108.585) (width 0.25) (layer "F.Cu") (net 1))
 (segment (start 140.716 108.585) (end 141.226 109.095) (width 0.25) (layer "F.Cu") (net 1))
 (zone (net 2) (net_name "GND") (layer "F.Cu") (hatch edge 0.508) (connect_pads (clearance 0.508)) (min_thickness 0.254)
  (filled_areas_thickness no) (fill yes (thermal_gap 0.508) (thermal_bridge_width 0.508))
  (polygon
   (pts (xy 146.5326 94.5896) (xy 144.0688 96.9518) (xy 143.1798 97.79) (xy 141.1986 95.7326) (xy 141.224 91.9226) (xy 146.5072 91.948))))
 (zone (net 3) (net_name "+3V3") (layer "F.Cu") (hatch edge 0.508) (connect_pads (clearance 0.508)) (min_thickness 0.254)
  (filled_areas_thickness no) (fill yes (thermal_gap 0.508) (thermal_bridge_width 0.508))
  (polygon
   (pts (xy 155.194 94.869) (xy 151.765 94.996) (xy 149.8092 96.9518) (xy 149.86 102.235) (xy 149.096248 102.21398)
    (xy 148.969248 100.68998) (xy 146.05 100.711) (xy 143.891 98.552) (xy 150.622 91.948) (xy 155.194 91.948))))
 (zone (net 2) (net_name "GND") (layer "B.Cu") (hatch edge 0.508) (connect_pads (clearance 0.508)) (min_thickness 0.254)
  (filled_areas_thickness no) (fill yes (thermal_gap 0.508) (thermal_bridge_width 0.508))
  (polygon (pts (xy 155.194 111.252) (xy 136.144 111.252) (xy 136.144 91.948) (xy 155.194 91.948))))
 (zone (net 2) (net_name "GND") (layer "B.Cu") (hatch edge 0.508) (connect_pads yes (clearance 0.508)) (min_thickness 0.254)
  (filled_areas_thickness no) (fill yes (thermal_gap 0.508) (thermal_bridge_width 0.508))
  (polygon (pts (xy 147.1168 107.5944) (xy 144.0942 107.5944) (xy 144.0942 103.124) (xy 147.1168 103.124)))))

